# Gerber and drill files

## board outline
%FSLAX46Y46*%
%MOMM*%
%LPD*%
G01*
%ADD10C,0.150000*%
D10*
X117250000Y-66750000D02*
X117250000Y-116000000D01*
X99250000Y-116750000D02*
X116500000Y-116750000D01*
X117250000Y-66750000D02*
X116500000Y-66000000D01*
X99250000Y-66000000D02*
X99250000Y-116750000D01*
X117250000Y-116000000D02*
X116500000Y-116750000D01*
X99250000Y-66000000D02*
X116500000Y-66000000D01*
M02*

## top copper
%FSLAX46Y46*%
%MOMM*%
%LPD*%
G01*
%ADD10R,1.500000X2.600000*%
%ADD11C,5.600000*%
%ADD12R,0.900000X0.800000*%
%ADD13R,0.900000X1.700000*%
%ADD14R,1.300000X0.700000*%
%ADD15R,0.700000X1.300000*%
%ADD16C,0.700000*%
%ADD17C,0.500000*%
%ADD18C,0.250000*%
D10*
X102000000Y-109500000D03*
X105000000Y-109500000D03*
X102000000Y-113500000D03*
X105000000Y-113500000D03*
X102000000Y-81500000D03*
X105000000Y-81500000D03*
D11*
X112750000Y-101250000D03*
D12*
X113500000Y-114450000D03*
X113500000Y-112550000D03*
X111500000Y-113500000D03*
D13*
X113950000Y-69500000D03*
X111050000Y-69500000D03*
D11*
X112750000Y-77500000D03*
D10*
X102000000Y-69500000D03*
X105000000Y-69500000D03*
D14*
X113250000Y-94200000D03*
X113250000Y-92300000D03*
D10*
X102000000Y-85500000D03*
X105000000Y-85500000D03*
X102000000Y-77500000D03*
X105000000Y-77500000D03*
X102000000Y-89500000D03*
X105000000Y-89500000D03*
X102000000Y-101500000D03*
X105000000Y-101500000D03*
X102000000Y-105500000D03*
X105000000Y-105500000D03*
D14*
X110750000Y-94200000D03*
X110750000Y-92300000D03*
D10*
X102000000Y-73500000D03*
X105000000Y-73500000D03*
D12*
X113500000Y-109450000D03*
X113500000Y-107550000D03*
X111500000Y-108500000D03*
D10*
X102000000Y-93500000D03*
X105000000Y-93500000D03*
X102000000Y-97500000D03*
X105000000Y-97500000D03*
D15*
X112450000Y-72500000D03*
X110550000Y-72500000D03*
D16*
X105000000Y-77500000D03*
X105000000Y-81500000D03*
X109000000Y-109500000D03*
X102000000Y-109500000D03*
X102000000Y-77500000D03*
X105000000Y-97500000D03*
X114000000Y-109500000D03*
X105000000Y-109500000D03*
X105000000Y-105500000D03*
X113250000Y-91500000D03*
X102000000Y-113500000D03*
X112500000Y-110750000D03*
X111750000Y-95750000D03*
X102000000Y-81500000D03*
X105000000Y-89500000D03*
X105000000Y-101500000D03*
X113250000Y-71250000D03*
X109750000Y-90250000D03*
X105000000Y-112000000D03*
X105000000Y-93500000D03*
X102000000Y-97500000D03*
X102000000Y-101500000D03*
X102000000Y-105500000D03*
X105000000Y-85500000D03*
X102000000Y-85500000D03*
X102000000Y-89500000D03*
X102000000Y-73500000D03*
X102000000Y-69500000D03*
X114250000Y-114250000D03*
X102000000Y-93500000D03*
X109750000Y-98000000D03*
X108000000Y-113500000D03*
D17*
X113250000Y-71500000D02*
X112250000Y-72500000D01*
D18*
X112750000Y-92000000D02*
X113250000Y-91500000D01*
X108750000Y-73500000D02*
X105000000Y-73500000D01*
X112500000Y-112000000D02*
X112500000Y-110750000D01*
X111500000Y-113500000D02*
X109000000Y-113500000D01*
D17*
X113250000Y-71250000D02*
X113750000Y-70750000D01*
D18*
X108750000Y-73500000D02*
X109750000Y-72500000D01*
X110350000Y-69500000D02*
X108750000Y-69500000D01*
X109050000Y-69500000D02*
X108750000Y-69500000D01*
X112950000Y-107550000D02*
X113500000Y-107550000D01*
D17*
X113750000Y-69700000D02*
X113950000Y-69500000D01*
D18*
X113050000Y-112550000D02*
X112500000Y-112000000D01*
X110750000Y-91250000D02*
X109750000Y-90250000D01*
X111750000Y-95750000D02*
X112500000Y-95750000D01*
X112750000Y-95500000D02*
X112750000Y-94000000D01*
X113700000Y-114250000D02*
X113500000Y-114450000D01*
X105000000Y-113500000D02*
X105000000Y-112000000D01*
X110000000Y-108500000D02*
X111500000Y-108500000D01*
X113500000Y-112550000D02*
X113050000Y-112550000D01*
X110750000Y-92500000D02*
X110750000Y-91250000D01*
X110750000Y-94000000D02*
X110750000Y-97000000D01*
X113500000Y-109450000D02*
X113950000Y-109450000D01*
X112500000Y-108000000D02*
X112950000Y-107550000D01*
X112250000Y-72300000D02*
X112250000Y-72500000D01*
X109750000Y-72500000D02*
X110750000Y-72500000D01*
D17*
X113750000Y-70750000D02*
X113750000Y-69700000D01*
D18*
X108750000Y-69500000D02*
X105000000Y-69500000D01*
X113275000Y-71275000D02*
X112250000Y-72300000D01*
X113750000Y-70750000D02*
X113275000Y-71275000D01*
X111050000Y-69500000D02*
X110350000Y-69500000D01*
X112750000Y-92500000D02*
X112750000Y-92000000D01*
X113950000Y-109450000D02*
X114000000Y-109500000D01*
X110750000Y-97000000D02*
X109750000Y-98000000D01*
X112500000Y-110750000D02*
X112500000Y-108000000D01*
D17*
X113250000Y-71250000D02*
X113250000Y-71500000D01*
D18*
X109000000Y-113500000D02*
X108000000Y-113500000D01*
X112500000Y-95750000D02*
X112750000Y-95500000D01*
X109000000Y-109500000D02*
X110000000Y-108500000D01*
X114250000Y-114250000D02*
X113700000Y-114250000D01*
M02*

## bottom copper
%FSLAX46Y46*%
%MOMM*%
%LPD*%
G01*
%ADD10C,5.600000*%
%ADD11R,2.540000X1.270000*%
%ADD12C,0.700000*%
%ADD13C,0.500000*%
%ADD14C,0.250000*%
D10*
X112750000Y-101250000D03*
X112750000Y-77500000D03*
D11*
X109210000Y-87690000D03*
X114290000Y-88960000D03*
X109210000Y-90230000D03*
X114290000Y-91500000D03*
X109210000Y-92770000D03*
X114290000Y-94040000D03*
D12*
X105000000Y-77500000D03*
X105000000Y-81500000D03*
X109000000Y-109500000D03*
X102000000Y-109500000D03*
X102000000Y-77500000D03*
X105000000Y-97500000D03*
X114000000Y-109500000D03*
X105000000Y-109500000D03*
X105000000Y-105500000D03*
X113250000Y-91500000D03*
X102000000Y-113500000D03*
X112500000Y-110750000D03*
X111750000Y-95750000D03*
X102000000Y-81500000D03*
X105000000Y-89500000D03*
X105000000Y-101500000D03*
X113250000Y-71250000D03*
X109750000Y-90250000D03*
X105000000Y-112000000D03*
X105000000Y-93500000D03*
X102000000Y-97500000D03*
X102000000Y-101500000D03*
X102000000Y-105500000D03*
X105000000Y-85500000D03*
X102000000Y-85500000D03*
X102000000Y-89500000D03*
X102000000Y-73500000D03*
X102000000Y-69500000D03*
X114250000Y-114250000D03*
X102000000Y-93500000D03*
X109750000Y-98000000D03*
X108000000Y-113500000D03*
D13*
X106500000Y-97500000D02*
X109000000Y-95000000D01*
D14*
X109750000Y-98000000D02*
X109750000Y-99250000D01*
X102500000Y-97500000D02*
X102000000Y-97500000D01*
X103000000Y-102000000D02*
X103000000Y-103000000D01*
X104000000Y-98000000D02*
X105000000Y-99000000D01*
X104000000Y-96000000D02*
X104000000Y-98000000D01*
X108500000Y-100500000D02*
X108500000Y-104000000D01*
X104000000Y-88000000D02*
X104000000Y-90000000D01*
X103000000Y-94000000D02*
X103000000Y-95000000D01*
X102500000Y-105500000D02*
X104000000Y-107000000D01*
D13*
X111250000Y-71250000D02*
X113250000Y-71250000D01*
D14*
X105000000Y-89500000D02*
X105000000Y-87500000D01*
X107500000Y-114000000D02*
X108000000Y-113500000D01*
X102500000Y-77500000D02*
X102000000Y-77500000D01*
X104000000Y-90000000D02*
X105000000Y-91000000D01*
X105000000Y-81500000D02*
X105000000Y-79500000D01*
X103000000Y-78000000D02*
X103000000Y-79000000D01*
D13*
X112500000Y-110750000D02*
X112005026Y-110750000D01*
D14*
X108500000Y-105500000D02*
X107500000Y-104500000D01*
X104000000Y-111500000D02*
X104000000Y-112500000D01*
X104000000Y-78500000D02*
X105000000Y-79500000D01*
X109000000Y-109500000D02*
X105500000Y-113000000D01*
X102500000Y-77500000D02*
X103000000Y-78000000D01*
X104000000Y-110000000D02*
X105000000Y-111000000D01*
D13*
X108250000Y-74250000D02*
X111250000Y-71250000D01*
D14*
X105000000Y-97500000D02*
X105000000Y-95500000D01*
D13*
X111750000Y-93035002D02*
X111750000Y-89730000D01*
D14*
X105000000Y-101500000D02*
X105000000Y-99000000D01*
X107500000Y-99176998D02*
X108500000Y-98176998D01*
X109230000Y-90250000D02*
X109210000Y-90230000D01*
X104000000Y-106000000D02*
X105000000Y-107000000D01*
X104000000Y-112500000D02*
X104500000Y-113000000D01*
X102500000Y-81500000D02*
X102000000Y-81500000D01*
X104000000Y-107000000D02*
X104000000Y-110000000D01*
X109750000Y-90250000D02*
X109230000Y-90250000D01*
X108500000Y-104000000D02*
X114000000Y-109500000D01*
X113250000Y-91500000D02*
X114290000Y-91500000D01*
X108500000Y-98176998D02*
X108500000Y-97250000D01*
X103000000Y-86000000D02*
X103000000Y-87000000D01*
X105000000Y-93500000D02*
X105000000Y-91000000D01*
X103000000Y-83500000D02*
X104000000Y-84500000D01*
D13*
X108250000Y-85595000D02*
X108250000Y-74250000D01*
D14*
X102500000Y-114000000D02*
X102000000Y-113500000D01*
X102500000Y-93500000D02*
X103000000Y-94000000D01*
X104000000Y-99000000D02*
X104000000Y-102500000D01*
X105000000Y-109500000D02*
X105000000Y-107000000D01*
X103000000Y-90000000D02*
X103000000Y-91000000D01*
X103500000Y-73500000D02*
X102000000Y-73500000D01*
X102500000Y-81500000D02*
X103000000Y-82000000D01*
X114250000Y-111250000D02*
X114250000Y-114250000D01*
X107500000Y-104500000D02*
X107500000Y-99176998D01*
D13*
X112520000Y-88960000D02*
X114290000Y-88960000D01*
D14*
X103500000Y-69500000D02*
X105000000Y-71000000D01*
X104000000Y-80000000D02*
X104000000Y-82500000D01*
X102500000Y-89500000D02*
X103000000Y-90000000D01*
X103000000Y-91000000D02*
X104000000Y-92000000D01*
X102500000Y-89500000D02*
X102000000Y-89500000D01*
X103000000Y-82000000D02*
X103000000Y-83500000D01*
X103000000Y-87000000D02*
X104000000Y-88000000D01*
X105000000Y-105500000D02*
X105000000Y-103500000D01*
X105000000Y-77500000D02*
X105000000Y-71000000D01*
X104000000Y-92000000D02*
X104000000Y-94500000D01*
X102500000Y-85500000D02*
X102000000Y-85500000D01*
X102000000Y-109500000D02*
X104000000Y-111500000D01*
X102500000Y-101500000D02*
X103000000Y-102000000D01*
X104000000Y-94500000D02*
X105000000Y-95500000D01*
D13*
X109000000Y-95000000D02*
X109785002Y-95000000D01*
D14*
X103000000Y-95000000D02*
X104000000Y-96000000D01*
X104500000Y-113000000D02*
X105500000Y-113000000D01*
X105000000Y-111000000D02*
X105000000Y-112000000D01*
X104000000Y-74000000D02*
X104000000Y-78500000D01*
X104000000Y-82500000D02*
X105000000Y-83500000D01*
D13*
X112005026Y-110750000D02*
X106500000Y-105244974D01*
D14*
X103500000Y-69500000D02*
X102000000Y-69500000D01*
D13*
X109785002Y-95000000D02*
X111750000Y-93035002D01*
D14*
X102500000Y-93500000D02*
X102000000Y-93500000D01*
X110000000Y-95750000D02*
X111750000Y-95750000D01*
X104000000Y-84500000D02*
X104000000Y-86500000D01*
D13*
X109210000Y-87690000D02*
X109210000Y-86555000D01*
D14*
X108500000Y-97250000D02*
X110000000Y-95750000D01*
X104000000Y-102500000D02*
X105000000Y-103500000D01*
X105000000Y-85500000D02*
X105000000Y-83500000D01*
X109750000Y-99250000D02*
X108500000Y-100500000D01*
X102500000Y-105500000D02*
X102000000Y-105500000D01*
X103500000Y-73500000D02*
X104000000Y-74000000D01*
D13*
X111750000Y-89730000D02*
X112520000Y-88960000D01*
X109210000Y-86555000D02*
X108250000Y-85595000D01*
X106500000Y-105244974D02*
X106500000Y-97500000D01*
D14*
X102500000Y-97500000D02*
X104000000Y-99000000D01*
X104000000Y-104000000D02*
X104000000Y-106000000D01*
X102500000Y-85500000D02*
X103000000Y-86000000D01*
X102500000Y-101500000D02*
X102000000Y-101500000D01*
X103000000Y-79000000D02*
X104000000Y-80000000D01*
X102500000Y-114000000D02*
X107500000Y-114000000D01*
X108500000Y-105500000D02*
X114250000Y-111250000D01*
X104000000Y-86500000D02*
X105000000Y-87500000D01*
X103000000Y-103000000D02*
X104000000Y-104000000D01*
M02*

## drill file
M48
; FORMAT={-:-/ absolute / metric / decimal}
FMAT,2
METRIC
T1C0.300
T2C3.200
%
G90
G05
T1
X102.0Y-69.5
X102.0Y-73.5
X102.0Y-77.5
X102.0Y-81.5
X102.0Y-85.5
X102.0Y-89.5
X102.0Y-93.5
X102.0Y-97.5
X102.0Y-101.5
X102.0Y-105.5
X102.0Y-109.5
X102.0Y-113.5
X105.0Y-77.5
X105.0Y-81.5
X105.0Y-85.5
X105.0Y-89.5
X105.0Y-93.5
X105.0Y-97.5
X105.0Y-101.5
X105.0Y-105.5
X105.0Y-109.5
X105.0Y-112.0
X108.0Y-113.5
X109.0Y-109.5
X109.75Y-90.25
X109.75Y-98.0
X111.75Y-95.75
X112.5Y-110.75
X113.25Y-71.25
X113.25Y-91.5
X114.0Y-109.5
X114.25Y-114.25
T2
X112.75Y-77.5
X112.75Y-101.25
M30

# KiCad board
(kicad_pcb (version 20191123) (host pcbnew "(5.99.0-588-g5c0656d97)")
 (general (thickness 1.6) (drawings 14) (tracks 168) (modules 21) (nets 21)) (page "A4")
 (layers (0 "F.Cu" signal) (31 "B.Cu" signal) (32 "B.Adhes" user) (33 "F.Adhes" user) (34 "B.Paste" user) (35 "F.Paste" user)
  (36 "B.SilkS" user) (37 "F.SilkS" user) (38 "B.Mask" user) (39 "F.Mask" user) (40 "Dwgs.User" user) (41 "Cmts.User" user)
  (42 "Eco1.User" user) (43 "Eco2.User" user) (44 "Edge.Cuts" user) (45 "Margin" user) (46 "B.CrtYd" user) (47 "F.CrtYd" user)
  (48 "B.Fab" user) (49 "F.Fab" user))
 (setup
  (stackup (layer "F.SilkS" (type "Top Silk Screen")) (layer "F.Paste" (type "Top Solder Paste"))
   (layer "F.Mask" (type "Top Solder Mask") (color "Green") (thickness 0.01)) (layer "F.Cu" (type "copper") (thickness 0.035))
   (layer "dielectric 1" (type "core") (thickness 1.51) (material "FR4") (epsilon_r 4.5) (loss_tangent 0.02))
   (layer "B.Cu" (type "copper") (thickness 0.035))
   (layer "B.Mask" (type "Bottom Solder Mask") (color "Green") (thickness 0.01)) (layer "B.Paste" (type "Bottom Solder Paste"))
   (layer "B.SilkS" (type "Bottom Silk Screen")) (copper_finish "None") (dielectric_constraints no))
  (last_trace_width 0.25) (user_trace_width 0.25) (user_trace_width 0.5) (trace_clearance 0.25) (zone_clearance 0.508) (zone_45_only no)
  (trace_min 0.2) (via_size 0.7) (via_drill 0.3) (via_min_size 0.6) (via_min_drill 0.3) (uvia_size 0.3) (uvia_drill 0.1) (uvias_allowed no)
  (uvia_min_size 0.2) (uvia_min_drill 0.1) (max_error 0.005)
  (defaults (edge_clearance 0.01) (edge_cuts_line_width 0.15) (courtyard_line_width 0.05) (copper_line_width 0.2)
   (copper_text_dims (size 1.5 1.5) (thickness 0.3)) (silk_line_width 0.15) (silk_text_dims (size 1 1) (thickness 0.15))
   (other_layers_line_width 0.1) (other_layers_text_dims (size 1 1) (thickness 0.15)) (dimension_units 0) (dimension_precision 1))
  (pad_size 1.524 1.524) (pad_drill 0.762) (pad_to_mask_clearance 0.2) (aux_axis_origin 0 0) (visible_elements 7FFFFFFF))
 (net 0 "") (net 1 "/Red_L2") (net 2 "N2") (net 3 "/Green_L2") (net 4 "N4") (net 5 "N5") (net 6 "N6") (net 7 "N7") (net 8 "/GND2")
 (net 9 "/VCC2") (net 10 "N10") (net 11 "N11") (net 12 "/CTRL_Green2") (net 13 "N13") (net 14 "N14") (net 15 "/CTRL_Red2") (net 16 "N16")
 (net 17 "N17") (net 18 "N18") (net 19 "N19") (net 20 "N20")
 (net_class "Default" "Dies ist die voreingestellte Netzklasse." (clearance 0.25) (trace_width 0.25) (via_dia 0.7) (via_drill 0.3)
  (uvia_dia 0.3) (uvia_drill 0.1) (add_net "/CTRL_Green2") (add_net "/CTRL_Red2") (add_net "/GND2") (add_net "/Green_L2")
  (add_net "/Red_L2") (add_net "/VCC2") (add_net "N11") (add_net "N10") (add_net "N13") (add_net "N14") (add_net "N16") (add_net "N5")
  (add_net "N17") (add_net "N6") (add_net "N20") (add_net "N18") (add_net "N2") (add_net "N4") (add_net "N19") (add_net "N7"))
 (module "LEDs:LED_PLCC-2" (layer "F.Cu") (at 103.5 109.5)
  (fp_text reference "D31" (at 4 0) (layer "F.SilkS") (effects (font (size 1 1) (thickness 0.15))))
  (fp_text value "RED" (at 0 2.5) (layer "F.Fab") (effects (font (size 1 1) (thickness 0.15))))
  (pad "1" smd rect (at -1.5 0) (size 1.5 2.6) (layers "F.Cu" "F.Paste" "F.Mask") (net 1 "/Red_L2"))
  (pad "2" smd rect (at 1.5 0) (size 1.5 2.6) (layers "F.Cu" "F.Paste" "F.Mask") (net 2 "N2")))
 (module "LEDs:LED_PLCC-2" (layer "F.Cu") (at 103.5 113.5)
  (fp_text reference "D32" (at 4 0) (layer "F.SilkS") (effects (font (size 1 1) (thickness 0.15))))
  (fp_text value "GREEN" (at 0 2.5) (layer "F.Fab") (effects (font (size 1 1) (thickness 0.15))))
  (pad "1" smd rect (at -1.5 0) (size 1.5 2.6) (layers "F.Cu" "F.Paste" "F.Mask") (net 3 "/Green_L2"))
  (pad "2" smd rect (at 1.5 0) (size 1.5 2.6) (layers "F.Cu" "F.Paste" "F.Mask") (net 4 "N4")))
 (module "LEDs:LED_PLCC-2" (layer "F.Cu") (at 103.5 81.5)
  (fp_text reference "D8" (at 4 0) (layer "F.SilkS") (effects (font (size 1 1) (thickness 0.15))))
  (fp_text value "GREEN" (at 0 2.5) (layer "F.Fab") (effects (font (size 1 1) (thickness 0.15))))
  (pad "1" smd rect (at -1.5 0) (size 1.5 2.6) (layers "F.Cu" "F.Paste" "F.Mask") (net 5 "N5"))
  (pad "2" smd rect (at 1.5 0) (size 1.5 2.6) (layers "F.Cu" "F.Paste" "F.Mask") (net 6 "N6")))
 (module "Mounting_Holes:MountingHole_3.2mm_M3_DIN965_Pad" (layer "F.Cu") (at 112.75 101.25)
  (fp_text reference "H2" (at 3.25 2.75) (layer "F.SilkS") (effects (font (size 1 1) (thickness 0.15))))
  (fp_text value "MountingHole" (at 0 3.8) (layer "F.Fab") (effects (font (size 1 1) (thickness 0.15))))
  (pad "1" thru_hole circle (at 0 0) (size 5.6 5.6) (drill 3.2) (layers *.Cu *.Mask)))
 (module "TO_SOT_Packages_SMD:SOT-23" (layer "F.Cu") (at 112.5 113.5 180)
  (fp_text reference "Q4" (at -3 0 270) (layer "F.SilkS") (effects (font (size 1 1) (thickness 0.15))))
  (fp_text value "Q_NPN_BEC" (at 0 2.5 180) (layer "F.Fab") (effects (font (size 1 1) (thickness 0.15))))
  (pad "1" smd rect (at -1 -0.95 180) (size 0.9 0.8) (layers "F.Cu" "F.Paste" "F.Mask") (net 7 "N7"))
  (pad "2" smd rect (at -1 0.95 180) (size 0.9 0.8) (layers "F.Cu" "F.Paste" "F.Mask") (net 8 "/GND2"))
  (pad "3" smd rect (at 1 0 180) (size 0.9 0.8) (layers "F.Cu" "F.Paste" "F.Mask") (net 3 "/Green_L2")))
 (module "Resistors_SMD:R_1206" (layer "F.Cu") (at 112.5 69.5 180)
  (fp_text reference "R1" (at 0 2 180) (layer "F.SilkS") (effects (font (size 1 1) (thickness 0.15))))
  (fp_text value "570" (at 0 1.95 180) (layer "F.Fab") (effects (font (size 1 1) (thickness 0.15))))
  (pad "1" smd rect (at -1.45 0 180) (size 0.9 1.7) (layers "F.Cu" "F.Paste" "F.Mask") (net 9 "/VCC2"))
  (pad "2" smd rect (at 1.45 0 180) (size 0.9 1.7) (layers "F.Cu" "F.Paste" "F.Mask") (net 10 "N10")))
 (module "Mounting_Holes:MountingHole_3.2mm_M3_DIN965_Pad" (layer "F.Cu") (at 112.75 77.5)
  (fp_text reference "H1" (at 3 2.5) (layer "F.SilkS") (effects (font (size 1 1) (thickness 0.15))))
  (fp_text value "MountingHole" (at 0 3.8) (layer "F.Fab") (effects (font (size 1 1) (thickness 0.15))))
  (pad "1" thru_hole circle (at 0 0) (size 5.6 5.6) (drill 3.2) (layers *.Cu *.Mask)))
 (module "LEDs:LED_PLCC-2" (layer "F.Cu") (at 103.5 69.5)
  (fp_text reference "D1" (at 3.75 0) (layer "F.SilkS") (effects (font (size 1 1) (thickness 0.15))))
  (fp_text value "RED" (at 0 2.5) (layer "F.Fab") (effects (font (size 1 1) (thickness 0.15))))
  (pad "1" smd rect (at -1.5 0) (size 1.5 2.6) (layers "F.Cu" "F.Paste" "F.Mask") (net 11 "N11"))
  (pad "2" smd rect (at 1.5 0) (size 1.5 2.6) (layers "F.Cu" "F.Paste" "F.Mask") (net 10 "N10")))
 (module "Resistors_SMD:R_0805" (layer "F.Cu") (at 113.25 93.25 90)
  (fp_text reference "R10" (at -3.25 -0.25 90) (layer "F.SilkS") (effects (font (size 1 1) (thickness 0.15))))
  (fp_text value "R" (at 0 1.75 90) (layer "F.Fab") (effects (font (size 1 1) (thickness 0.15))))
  (pad "1" smd rect (at -0.95 0 90) (size 0.7 1.3) (layers "F.Cu" "F.Paste" "F.Mask") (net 7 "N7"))
  (pad "2" smd rect (at 0.95 0 90) (size 0.7 1.3) (layers "F.Cu" "F.Paste" "F.Mask") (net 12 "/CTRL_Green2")))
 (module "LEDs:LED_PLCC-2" (layer "F.Cu") (at 103.5 85.5)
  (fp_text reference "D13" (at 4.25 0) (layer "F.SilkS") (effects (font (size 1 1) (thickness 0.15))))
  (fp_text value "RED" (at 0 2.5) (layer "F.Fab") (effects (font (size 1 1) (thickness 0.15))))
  (pad "1" smd rect (at -1.5 0) (size 1.5 2.6) (layers "F.Cu" "F.Paste" "F.Mask") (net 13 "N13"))
  (pad "2" smd rect (at 1.5 0) (size 1.5 2.6) (layers "F.Cu" "F.Paste" "F.Mask") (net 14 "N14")))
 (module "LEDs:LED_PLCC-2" (layer "F.Cu") (at 103.5 77.5)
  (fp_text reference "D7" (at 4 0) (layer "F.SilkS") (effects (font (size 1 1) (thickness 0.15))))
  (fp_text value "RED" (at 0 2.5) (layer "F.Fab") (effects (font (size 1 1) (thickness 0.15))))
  (pad "1" smd rect (at -1.5 0) (size 1.5 2.6) (layers "F.Cu" "F.Paste" "F.Mask") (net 14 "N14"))
  (pad "2" smd rect (at 1.5 0) (size 1.5 2.6) (layers "F.Cu" "F.Paste" "F.Mask") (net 11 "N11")))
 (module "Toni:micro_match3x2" (layer "B.Cu") (at 111.75 91.5 -90)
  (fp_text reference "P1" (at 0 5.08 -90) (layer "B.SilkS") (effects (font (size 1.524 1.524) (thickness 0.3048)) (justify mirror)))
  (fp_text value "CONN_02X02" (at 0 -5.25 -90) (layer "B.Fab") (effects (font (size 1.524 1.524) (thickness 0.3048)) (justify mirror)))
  (pad "1" smd rect (at -3.81 2.54 270) (size 1.27 2.54) (layers "B.Cu" "B.Paste" "B.Mask") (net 9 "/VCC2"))
  (pad "2" smd rect (at -2.54 -2.54 270) (size 1.27 2.54) (layers "B.Cu" "B.Paste" "B.Mask") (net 8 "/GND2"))
  (pad "3" smd rect (at -1.27 2.54 270) (size 1.27 2.54) (layers "B.Cu" "B.Paste" "B.Mask") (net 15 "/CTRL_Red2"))
  (pad "4" smd rect (at 0 -2.54 270) (size 1.27 2.54) (layers "B.Cu" "B.Paste" "B.Mask") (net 12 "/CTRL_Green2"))
  (pad "5" smd rect (at 1.27 2.54 270) (size 1.27 2.54) (layers "B.Cu" "B.Paste" "B.Mask"))
  (pad "6" smd rect (at 2.54 -2.54 270) (size 1.27 2.54) (layers "B.Cu" "B.Paste" "B.Mask")))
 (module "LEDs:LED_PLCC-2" (layer "F.Cu") (at 103.5 89.5)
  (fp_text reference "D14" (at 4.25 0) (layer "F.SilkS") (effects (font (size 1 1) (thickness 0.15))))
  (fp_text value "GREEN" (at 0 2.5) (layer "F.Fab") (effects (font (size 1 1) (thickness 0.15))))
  (pad "1" smd rect (at -1.5 0) (size 1.5 2.6) (layers "F.Cu" "F.Paste" "F.Mask") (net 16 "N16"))
  (pad "2" smd rect (at 1.5 0) (size 1.5 2.6) (layers "F.Cu" "F.Paste" "F.Mask") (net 5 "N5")))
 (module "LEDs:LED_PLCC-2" (layer "F.Cu") (at 103.5 101.5)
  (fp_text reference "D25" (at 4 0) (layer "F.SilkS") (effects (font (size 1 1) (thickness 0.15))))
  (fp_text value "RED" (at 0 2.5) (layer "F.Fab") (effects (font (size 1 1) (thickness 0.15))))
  (pad "1" smd rect (at -1.5 0) (size 1.5 2.6) (layers "F.Cu" "F.Paste" "F.Mask") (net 2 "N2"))
  (pad "2" smd rect (at 1.5 0) (size 1.5 2.6) (layers "F.Cu" "F.Paste" "F.Mask") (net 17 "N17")))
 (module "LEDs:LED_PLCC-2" (layer "F.Cu") (at 103.5 105.5)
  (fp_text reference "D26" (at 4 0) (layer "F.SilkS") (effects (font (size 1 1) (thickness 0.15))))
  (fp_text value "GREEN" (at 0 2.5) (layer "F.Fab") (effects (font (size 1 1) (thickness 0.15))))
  (pad "1" smd rect (at -1.5 0) (size 1.5 2.6) (layers "F.Cu" "F.Paste" "F.Mask") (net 4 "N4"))
  (pad "2" smd rect (at 1.5 0) (size 1.5 2.6) (layers "F.Cu" "F.Paste" "F.Mask") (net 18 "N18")))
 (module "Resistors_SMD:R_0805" (layer "F.Cu") (at 110.75 93.25 90)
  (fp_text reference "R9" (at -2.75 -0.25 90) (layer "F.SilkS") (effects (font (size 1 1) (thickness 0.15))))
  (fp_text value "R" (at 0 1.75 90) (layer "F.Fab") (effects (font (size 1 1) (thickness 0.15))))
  (pad "1" smd rect (at -0.95 0 90) (size 0.7 1.3) (layers "F.Cu" "F.Paste" "F.Mask") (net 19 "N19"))
  (pad "2" smd rect (at 0.95 0 90) (size 0.7 1.3) (layers "F.Cu" "F.Paste" "F.Mask") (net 15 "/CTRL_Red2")))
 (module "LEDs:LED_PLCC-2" (layer "F.Cu") (at 103.5 73.5)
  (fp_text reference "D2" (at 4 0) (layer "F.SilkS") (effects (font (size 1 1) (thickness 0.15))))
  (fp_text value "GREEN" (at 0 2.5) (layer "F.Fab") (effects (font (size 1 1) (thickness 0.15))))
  (pad "1" smd rect (at -1.5 0) (size 1.5 2.6) (layers "F.Cu" "F.Paste" "F.Mask") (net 6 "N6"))
  (pad "2" smd rect (at 1.5 0) (size 1.5 2.6) (layers "F.Cu" "F.Paste" "F.Mask") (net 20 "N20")))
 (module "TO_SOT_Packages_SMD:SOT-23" (layer "F.Cu") (at 112.5 108.5 180)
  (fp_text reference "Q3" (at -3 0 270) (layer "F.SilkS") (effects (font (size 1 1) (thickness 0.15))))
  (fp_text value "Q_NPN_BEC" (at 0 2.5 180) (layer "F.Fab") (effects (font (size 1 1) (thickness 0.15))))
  (pad "1" smd rect (at -1 -0.95 180) (size 0.9 0.8) (layers "F.Cu" "F.Paste" "F.Mask") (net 19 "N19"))
  (pad "2" smd rect (at -1 0.95 180) (size 0.9 0.8) (layers "F.Cu" "F.Paste" "F.Mask") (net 8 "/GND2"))
  (pad "3" smd rect (at 1 0 180) (size 0.9 0.8) (layers "F.Cu" "F.Paste" "F.Mask") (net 1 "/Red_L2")))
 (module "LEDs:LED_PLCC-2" (layer "F.Cu") (at 103.5 93.5)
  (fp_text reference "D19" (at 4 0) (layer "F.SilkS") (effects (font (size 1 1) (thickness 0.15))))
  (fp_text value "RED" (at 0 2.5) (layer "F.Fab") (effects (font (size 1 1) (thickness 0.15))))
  (pad "1" smd rect (at -1.5 0) (size 1.5 2.6) (layers "F.Cu" "F.Paste" "F.Mask") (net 17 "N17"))
  (pad "2" smd rect (at 1.5 0) (size 1.5 2.6) (layers "F.Cu" "F.Paste" "F.Mask") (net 13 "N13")))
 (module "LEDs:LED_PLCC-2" (layer "F.Cu") (at 103.5 97.5)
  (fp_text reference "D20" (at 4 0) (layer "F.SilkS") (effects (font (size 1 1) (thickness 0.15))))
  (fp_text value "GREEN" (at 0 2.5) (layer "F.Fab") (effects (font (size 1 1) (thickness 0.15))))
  (pad "1" smd rect (at -1.5 0) (size 1.5 2.6) (layers "F.Cu" "F.Paste" "F.Mask") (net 18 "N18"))
  (pad "2" smd rect (at 1.5 0) (size 1.5 2.6) (layers "F.Cu" "F.Paste" "F.Mask") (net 16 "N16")))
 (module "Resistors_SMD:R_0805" (layer "F.Cu") (at 111.5 72.5 180)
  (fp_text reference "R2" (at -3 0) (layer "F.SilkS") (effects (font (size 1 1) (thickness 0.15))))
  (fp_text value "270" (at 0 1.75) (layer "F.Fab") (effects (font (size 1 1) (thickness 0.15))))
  (pad "1" smd rect (at -0.95 0 180) (size 0.7 1.3) (layers "F.Cu" "F.Paste" "F.Mask") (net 9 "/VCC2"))
  (pad "2" smd rect (at 0.95 0 180) (size 0.7 1.3) (layers "F.Cu" "F.Paste" "F.Mask") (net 20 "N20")))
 (gr_line (start 117.25 66.75) (end 117.25 116) (layer "Edge.Cuts") (width 0.15))
 (gr_line (start 99.25 116.75) (end 116.5 116.75) (layer "Edge.Cuts") (width 0.15))
 (gr_line (start 117.25 66.75) (end 116.5 66) (layer "Edge.Cuts") (width 0.15))
 (gr_line (start 99.25 66) (end 99.25 116.75) (layer "Edge.Cuts") (width 0.15))
 (gr_line (start 117.25 116) (end 116.5 116.75) (layer "Edge.Cuts") (width 0.15))
 (gr_line (start 99.25 66) (end 116.5 66) (layer "Edge.Cuts") (width 0.15))
 (via (at 105 77.5) (size 0.7) (drill 0.3) (layers "F.Cu" "B.Cu") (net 11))
 (segment (start 113.25 71.5) (end 112.25 72.5) (width 0.5) (layer "F.Cu") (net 9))
 (segment (start 106.5 97.5) (end 109 95) (width 0.5) (layer "B.Cu") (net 8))
 (segment (start 109.75 98) (end 109.75 99.25) (width 0.25) (layer "B.Cu") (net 19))
 (segment (start 102.5 97.5) (end 102 97.5) (width 0.25) (layer "B.Cu") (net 18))
 (segment (start 103 102) (end 103 103) (width 0.25) (layer "B.Cu") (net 2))
 (segment (start 112.75 92) (end 113.25 91.5) (width 0.25) (layer "F.Cu") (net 12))
 (segment (start 108.75 73.5) (end 105 73.5) (width 0.25) (layer "F.Cu") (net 20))
 (segment (start 104 98) (end 105 99) (width 0.25) (layer "B.Cu") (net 17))
 (segment (start 104 96) (end 104 98) (width 0.25) (layer "B.Cu") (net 17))
 (segment (start 108.5 100.5) (end 108.5 104) (width 0.25) (layer "B.Cu") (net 19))
 (segment (start 112.5 112) (end 112.5 110.75) (width 0.25) (layer "F.Cu") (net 8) (status 8000))
 (segment (start 104 88) (end 104 90) (width 0.25) (layer "B.Cu") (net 13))
 (segment (start 103 94) (end 103 95) (width 0.25) (layer "B.Cu") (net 17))
 (segment (start 102.5 105.5) (end 104 107) (width 0.25) (layer "B.Cu") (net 4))
 (segment (start 111.5 113.5) (end 109 113.5) (width 0.25) (layer "F.Cu") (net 3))
 (segment (start 111.25 71.25) (end 113.25 71.25) (width 0.5) (layer "B.Cu") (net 9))
 (segment (start 113.25 71.25) (end 113.75 70.75) (width 0.5) (layer "F.Cu") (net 9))
 (via (at 105 81.5) (size 0.7) (drill 0.3) (layers "F.Cu" "B.Cu") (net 6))
 (segment (start 105 89.5) (end 105 87.5) (width 0.25) (layer "B.Cu") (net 5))
 (segment (start 108.75 73.5) (end 109.75 72.5) (width 0.25) (layer "F.Cu") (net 20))
 (segment (start 110.35 69.5) (end 108.75 69.5) (width 0.25) (layer "F.Cu") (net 10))
 (segment (start 109.05 69.5) (end 108.75 69.5) (width 0.25) (layer "F.Cu") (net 10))
 (segment (start 112.95 107.55) (end 113.5 107.55) (width 0.25) (layer "F.Cu") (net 8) (status 8000))
 (segment (start 113.75 69.7) (end 113.95 69.5) (width 0.5) (layer "F.Cu") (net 9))
 (segment (start 107.5 114) (end 108 113.5) (width 0.25) (layer "B.Cu") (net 3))
 (segment (start 113.05 112.55) (end 112.5 112) (width 0.25) (layer "F.Cu") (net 8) (status 8000))
 (segment (start 102.5 77.5) (end 102 77.5) (width 0.25) (layer "B.Cu") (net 14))
 (segment (start 104 90) (end 105 91) (width 0.25) (layer "B.Cu") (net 13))
 (segment (start 110.75 91.25) (end 109.75 90.25) (width 0.25) (layer "F.Cu") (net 15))
 (segment (start 111.75 95.75) (end 112.5 95.75) (width 0.25) (layer "F.Cu") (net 7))
 (segment (start 105 81.5) (end 105 79.5) (width 0.25) (layer "B.Cu") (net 6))
 (segment (start 112.75 95.5) (end 112.75 94) (width 0.25) (layer "F.Cu") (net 7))
 (segment (start 103 78) (end 103 79) (width 0.25) (layer "B.Cu") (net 14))
 (segment (start 112.5 110.75) (end 112.005026 110.75) (width 0.5) (layer "B.Cu") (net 8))
 (via (at 109 109.5) (size 0.7) (drill 0.3) (layers "F.Cu" "B.Cu") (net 1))
 (via (at 102 109.5) (size 0.7) (drill 0.3) (layers "F.Cu" "B.Cu") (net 1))
 (segment (start 108.5 105.5) (end 107.5 104.5) (width 0.25) (layer "B.Cu") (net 7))
 (segment (start 113.7 114.25) (end 113.5 114.45) (width 0.25) (layer "F.Cu") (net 7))
 (segment (start 104 111.5) (end 104 112.5) (width 0.25) (layer "B.Cu") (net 1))
 (segment (start 104 78.5) (end 105 79.5) (width 0.25) (layer "B.Cu") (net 6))
 (via (at 102 77.5) (size 0.7) (drill 0.3) (layers "F.Cu" "B.Cu") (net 14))
 (segment (start 109 109.5) (end 105.5 113) (width 0.25) (layer "B.Cu") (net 1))
 (segment (start 102.5 77.5) (end 103 78) (width 0.25) (layer "B.Cu") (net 14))
 (segment (start 104 110) (end 105 111) (width 0.25) (layer "B.Cu") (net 4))
 (segment (start 108.25 74.25) (end 111.25 71.25) (width 0.5) (layer "B.Cu") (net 9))
 (segment (start 105 113.5) (end 105 112) (width 0.25) (layer "F.Cu") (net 4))
 (segment (start 110 108.5) (end 111.5 108.5) (width 0.25) (layer "F.Cu") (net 1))
 (via (at 105 97.5) (size 0.7) (drill 0.3) (layers "F.Cu" "B.Cu") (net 16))
 (via (at 114 109.5) (size 0.7) (drill 0.3) (layers "F.Cu" "B.Cu") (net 19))
 (segment (start 105 97.5) (end 105 95.5) (width 0.25) (layer "B.Cu") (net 16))
 (via (at 105 109.5) (size 0.7) (drill 0.3) (layers "F.Cu" "B.Cu") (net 2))
 (segment (start 111.75 93.035002) (end 111.75 89.73) (width 0.5) (layer "B.Cu") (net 8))
 (segment (start 113.5 112.55) (end 113.05 112.55) (width 0.25) (layer "F.Cu") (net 8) (status 8000))
 (via (at 105 105.5) (size 0.7) (drill 0.3) (layers "F.Cu" "B.Cu") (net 18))
 (segment (start 105 101.5) (end 105 99) (width 0.25) (layer "B.Cu") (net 17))
 (segment (start 107.5 99.176998) (end 108.5 98.176998) (width 0.25) (layer "B.Cu") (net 7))
 (segment (start 110.75 92.5) (end 110.75 91.25) (width 0.25) (layer "F.Cu") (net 15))
 (segment (start 110.75 94) (end 110.75 97) (width 0.25) (layer "F.Cu") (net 19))
 (segment (start 109.23 90.25) (end 109.21 90.23) (width 0.25) (layer "B.Cu") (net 15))
 (segment (start 113.5 109.45) (end 113.95 109.45) (width 0.25) (layer "F.Cu") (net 19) (status C00000))
 (segment (start 104 106) (end 105 107) (width 0.25) (layer "B.Cu") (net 2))
 (segment (start 104 112.5) (end 104.5 113) (width 0.25) (layer "B.Cu") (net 1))
 (segment (start 102.5 81.5) (end 102 81.5) (width 0.25) (layer "B.Cu") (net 5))
 (via (at 113.25 91.5) (size 0.7) (drill 0.3) (layers "F.Cu" "B.Cu") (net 12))
 (via (at 102 113.5) (size 0.7) (drill 0.3) (layers "F.Cu" "B.Cu") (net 3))
 (segment (start 104 107) (end 104 110) (width 0.25) (layer "B.Cu") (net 4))
 (segment (start 109.75 90.25) (end 109.23 90.25) (width 0.25) (layer "B.Cu") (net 15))
 (via (at 112.5 110.75) (size 0.7) (drill 0.3) (layers "F.Cu" "B.Cu") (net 8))
 (segment (start 108.5 104) (end 114 109.5) (width 0.25) (layer "B.Cu") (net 19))
 (via (at 111.75 95.75) (size 0.7) (drill 0.3) (layers "F.Cu" "B.Cu") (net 7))
 (segment (start 113.25 91.5) (end 114.29 91.5) (width 0.25) (layer "B.Cu") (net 12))
 (segment (start 108.5 98.176998) (end 108.5 97.25) (width 0.25) (layer "B.Cu") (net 7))
 (segment (start 103 86) (end 103 87) (width 0.25) (layer "B.Cu") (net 13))
 (segment (start 105 93.5) (end 105 91) (width 0.25) (layer "B.Cu") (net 13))
 (segment (start 103 83.5) (end 104 84.5) (width 0.25) (layer "B.Cu") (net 5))
 (segment (start 108.25 85.595) (end 108.25 74.25) (width 0.5) (layer "B.Cu") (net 9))
 (segment (start 112.5 108) (end 112.95 107.55) (width 0.25) (layer "F.Cu") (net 8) (status 8000))
 (segment (start 112.25 72.3) (end 112.25 72.5) (width 0.25) (layer "F.Cu") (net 9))
 (segment (start 102.5 114) (end 102 113.5) (width 0.25) (layer "B.Cu") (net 3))
 (segment (start 102.5 93.5) (end 103 94) (width 0.25) (layer "B.Cu") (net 17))
 (segment (start 109.75 72.5) (end 110.75 72.5) (width 0.25) (layer "F.Cu") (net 20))
 (segment (start 104 99) (end 104 102.5) (width 0.25) (layer "B.Cu") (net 18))
 (segment (start 113.75 70.75) (end 113.75 69.7) (width 0.5) (layer "F.Cu") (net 9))
 (segment (start 105 109.5) (end 105 107) (width 0.25) (layer "B.Cu") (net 2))
 (segment (start 103 90) (end 103 91) (width 0.25) (layer "B.Cu") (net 16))
 (segment (start 103.5 73.5) (end 102 73.5) (width 0.25) (layer "B.Cu") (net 6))
 (segment (start 102.5 81.5) (end 103 82) (width 0.25) (layer "B.Cu") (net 5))
 (via (at 102 81.5) (size 0.7) (drill 0.3) (layers "F.Cu" "B.Cu") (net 5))
 (via (at 105 89.5) (size 0.7) (drill 0.3) (layers "F.Cu" "B.Cu") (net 5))
 (segment (start 114.25 111.25) (end 114.25 114.25) (width 0.25) (layer "B.Cu") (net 7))
 (via (at 105 101.5) (size 0.7) (drill 0.3) (layers "F.Cu" "B.Cu") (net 17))
 (segment (start 107.5 104.5) (end 107.5 99.176998) (width 0.25) (layer "B.Cu") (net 7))
 (segment (start 112.52 88.96) (end 114.29 88.96) (width 0.5) (layer "B.Cu") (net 8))
 (via (at 113.25 71.25) (size 0.7) (drill 0.3) (layers "F.Cu" "B.Cu") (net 9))
 (segment (start 103.5 69.5) (end 105 71) (width 0.25) (layer "B.Cu") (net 11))
 (segment (start 104 80) (end 104 82.5) (width 0.25) (layer "B.Cu") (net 14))
 (segment (start 102.5 89.5) (end 103 90) (width 0.25) (layer "B.Cu") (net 16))
 (segment (start 103 91) (end 104 92) (width 0.25) (layer "B.Cu") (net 16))
 (segment (start 102.5 89.5) (end 102 89.5) (width 0.25) (layer "B.Cu") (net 16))
 (segment (start 108.75 69.5) (end 105 69.5) (width 0.25) (layer "F.Cu") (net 10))
 (segment (start 103 82) (end 103 83.5) (width 0.25) (layer "B.Cu") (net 5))
 (segment (start 113.275 71.275) (end 112.25 72.3) (width 0.25) (layer "F.Cu") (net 9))
 (segment (start 103 87) (end 104 88) (width 0.25) (layer "B.Cu") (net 13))
 (segment (start 105 105.5) (end 105 103.5) (width 0.25) (layer "B.Cu") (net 18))
 (via (at 109.75 90.25) (size 0.7) (drill 0.3) (layers "F.Cu" "B.Cu") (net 15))
 (segment (start 105 77.5) (end 105 71) (width 0.25) (layer "B.Cu") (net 11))
 (segment (start 113.75 70.75) (end 113.275 71.275) (width 0.25) (layer "F.Cu") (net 9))
 (segment (start 104 92) (end 104 94.5) (width 0.25) (layer "B.Cu") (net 16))
 (segment (start 102.5 85.5) (end 102 85.5) (width 0.25) (layer "B.Cu") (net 13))
 (segment (start 102 109.5) (end 104 111.5) (width 0.25) (layer "B.Cu") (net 1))
 (segment (start 102.5 101.5) (end 103 102) (width 0.25) (layer "B.Cu") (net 2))
 (segment (start 104 94.5) (end 105 95.5) (width 0.25) (layer "B.Cu") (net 16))
 (segment (start 109 95) (end 109.785002 95) (width 0.5) (layer "B.Cu") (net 8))
 (via (at 105 112) (size 0.7) (drill 0.3) (layers "F.Cu" "B.Cu") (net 4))
 (segment (start 103 95) (end 104 96) (width 0.25) (layer "B.Cu") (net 17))
 (segment (start 104.5 113) (end 105.5 113) (width 0.25) (layer "B.Cu") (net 1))
 (segment (start 105 111) (end 105 112) (width 0.25) (layer "B.Cu") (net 4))
 (segment (start 104 74) (end 104 78.5) (width 0.25) (layer "B.Cu") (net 6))
 (segment (start 111.05 69.5) (end 110.35 69.5) (width 0.25) (layer "F.Cu") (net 10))
 (segment (start 112.75 92.5) (end 112.75 92) (width 0.25) (layer "F.Cu") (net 12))
 (segment (start 104 82.5) (end 105 83.5) (width 0.25) (layer "B.Cu") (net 14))
 (segment (start 112.005026 110.75) (end 106.5 105.244974) (width 0.5) (layer "B.Cu") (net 8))
 (segment (start 103.5 69.5) (end 102 69.5) (width 0.25) (layer "B.Cu") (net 11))
 (segment (start 109.785002 95) (end 111.75 93.035002) (width 0.5) (layer "B.Cu") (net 8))
 (via (at 105 93.5) (size 0.7) (drill 0.3) (layers "F.Cu" "B.Cu") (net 13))
 (segment (start 102.5 93.5) (end 102 93.5) (width 0.25) (layer "B.Cu") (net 17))
 (segment (start 110 95.75) (end 111.75 95.75) (width 0.25) (layer "B.Cu") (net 7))
 (segment (start 104 84.5) (end 104 86.5) (width 0.25) (layer "B.Cu") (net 5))
 (segment (start 109.21 87.69) (end 109.21 86.555) (width 0.5) (layer "B.Cu") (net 9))
 (via (at 102 97.5) (size 0.7) (drill 0.3) (layers "F.Cu" "B.Cu") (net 18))
 (via (at 102 101.5) (size 0.7) (drill 0.3) (layers "F.Cu" "B.Cu") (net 2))
 (via (at 102 105.5) (size 0.7) (drill 0.3) (layers "F.Cu" "B.Cu") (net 4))
 (segment (start 108.5 97.25) (end 110 95.75) (width 0.25) (layer "B.Cu") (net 7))
 (segment (start 113.95 109.45) (end 114 109.5) (width 0.25) (layer "F.Cu") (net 19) (status 400000))
 (segment (start 110.75 97) (end 109.75 98) (width 0.25) (layer "F.Cu") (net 19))
 (via (at 105 85.5) (size 0.7) (drill 0.3) (layers "F.Cu" "B.Cu") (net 14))
 (segment (start 112.5 110.75) (end 112.5 108) (width 0.25) (layer "F.Cu") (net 8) (status 8000))
 (segment (start 113.25 71.25) (end 113.25 71.5) (width 0.5) (layer "F.Cu") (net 9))
 (segment (start 104 102.5) (end 105 103.5) (width 0.25) (layer "B.Cu") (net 18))
 (segment (start 105 85.5) (end 105 83.5) (width 0.25) (layer "B.Cu") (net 14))
 (segment (start 109 113.5) (end 108 113.5) (width 0.25) (layer "F.Cu") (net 3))
 (via (at 102 85.5) (size 0.7) (drill 0.3) (layers "F.Cu" "B.Cu") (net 13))
 (segment (start 109.75 99.25) (end 108.5 100.5) (width 0.25) (layer "B.Cu") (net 19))
 (segment (start 102.5 105.5) (end 102 105.5) (width 0.25) (layer "B.Cu") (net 4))
 (segment (start 103.5 73.5) (end 104 74) (width 0.25) (layer "B.Cu") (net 6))
 (via (at 102 89.5) (size 0.7) (drill 0.3) (layers "F.Cu" "B.Cu") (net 16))
 (segment (start 111.75 89.73) (end 112.52 88.96) (width 0.5) (layer "B.Cu") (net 8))
 (segment (start 109.21 86.555) (end 108.25 85.595) (width 0.5) (layer "B.Cu") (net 9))
 (segment (start 106.5 105.244974) (end 106.5 97.5) (width 0.5) (layer "B.Cu") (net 8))
 (segment (start 102.5 97.5) (end 104 99) (width 0.25) (layer "B.Cu") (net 18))
 (via (at 102 73.5) (size 0.7) (drill 0.3) (layers "F.Cu" "B.Cu") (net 6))
 (segment (start 104 104) (end 104 106) (width 0.25) (layer "B.Cu") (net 2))
 (segment (start 102.5 85.5) (end 103 86) (width 0.25) (layer "B.Cu") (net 13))
 (segment (start 102.5 101.5) (end 102 101.5) (width 0.25) (layer "B.Cu") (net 2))
 (via (at 102 69.5) (size 0.7) (drill 0.3) (layers "F.Cu" "B.Cu") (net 11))
 (segment (start 103 79) (end 104 80) (width 0.25) (layer "B.Cu") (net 14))
 (segment (start 102.5 114) (end 107.5 114) (width 0.25) (layer "B.Cu") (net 3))
 (segment (start 112.5 95.75) (end 112.75 95.5) (width 0.25) (layer "F.Cu") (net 7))
 (via (at 114.25 114.25) (size 0.7) (drill 0.3) (layers "F.Cu" "B.Cu") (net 7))
 (segment (start 108.5 105.5) (end 114.25 111.25) (width 0.25) (layer "B.Cu") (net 7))
 (segment (start 109 109.5) (end 110 108.5) (width 0.25) (layer "F.Cu") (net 1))
 (segment (start 104 86.5) (end 105 87.5) (width 0.25) (layer "B.Cu") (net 5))
 (segment (start 114.25 114.25) (end 113.7 114.25) (width 0.25) (layer "F.Cu") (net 7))
 (via (at 102 93.5) (size 0.7) (drill 0.3) (layers "F.Cu" "B.Cu") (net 17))
 (segment (start 103 103) (end 104 104) (width 0.25) (layer "B.Cu") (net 2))
 (via (at 109.75 98) (size 0.7) (drill 0.3) (layers "F.Cu" "B.Cu") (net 19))
 (via (at 108 113.5) (size 0.7) (drill 0.3) (layers "F.Cu" "B.Cu") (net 3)))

